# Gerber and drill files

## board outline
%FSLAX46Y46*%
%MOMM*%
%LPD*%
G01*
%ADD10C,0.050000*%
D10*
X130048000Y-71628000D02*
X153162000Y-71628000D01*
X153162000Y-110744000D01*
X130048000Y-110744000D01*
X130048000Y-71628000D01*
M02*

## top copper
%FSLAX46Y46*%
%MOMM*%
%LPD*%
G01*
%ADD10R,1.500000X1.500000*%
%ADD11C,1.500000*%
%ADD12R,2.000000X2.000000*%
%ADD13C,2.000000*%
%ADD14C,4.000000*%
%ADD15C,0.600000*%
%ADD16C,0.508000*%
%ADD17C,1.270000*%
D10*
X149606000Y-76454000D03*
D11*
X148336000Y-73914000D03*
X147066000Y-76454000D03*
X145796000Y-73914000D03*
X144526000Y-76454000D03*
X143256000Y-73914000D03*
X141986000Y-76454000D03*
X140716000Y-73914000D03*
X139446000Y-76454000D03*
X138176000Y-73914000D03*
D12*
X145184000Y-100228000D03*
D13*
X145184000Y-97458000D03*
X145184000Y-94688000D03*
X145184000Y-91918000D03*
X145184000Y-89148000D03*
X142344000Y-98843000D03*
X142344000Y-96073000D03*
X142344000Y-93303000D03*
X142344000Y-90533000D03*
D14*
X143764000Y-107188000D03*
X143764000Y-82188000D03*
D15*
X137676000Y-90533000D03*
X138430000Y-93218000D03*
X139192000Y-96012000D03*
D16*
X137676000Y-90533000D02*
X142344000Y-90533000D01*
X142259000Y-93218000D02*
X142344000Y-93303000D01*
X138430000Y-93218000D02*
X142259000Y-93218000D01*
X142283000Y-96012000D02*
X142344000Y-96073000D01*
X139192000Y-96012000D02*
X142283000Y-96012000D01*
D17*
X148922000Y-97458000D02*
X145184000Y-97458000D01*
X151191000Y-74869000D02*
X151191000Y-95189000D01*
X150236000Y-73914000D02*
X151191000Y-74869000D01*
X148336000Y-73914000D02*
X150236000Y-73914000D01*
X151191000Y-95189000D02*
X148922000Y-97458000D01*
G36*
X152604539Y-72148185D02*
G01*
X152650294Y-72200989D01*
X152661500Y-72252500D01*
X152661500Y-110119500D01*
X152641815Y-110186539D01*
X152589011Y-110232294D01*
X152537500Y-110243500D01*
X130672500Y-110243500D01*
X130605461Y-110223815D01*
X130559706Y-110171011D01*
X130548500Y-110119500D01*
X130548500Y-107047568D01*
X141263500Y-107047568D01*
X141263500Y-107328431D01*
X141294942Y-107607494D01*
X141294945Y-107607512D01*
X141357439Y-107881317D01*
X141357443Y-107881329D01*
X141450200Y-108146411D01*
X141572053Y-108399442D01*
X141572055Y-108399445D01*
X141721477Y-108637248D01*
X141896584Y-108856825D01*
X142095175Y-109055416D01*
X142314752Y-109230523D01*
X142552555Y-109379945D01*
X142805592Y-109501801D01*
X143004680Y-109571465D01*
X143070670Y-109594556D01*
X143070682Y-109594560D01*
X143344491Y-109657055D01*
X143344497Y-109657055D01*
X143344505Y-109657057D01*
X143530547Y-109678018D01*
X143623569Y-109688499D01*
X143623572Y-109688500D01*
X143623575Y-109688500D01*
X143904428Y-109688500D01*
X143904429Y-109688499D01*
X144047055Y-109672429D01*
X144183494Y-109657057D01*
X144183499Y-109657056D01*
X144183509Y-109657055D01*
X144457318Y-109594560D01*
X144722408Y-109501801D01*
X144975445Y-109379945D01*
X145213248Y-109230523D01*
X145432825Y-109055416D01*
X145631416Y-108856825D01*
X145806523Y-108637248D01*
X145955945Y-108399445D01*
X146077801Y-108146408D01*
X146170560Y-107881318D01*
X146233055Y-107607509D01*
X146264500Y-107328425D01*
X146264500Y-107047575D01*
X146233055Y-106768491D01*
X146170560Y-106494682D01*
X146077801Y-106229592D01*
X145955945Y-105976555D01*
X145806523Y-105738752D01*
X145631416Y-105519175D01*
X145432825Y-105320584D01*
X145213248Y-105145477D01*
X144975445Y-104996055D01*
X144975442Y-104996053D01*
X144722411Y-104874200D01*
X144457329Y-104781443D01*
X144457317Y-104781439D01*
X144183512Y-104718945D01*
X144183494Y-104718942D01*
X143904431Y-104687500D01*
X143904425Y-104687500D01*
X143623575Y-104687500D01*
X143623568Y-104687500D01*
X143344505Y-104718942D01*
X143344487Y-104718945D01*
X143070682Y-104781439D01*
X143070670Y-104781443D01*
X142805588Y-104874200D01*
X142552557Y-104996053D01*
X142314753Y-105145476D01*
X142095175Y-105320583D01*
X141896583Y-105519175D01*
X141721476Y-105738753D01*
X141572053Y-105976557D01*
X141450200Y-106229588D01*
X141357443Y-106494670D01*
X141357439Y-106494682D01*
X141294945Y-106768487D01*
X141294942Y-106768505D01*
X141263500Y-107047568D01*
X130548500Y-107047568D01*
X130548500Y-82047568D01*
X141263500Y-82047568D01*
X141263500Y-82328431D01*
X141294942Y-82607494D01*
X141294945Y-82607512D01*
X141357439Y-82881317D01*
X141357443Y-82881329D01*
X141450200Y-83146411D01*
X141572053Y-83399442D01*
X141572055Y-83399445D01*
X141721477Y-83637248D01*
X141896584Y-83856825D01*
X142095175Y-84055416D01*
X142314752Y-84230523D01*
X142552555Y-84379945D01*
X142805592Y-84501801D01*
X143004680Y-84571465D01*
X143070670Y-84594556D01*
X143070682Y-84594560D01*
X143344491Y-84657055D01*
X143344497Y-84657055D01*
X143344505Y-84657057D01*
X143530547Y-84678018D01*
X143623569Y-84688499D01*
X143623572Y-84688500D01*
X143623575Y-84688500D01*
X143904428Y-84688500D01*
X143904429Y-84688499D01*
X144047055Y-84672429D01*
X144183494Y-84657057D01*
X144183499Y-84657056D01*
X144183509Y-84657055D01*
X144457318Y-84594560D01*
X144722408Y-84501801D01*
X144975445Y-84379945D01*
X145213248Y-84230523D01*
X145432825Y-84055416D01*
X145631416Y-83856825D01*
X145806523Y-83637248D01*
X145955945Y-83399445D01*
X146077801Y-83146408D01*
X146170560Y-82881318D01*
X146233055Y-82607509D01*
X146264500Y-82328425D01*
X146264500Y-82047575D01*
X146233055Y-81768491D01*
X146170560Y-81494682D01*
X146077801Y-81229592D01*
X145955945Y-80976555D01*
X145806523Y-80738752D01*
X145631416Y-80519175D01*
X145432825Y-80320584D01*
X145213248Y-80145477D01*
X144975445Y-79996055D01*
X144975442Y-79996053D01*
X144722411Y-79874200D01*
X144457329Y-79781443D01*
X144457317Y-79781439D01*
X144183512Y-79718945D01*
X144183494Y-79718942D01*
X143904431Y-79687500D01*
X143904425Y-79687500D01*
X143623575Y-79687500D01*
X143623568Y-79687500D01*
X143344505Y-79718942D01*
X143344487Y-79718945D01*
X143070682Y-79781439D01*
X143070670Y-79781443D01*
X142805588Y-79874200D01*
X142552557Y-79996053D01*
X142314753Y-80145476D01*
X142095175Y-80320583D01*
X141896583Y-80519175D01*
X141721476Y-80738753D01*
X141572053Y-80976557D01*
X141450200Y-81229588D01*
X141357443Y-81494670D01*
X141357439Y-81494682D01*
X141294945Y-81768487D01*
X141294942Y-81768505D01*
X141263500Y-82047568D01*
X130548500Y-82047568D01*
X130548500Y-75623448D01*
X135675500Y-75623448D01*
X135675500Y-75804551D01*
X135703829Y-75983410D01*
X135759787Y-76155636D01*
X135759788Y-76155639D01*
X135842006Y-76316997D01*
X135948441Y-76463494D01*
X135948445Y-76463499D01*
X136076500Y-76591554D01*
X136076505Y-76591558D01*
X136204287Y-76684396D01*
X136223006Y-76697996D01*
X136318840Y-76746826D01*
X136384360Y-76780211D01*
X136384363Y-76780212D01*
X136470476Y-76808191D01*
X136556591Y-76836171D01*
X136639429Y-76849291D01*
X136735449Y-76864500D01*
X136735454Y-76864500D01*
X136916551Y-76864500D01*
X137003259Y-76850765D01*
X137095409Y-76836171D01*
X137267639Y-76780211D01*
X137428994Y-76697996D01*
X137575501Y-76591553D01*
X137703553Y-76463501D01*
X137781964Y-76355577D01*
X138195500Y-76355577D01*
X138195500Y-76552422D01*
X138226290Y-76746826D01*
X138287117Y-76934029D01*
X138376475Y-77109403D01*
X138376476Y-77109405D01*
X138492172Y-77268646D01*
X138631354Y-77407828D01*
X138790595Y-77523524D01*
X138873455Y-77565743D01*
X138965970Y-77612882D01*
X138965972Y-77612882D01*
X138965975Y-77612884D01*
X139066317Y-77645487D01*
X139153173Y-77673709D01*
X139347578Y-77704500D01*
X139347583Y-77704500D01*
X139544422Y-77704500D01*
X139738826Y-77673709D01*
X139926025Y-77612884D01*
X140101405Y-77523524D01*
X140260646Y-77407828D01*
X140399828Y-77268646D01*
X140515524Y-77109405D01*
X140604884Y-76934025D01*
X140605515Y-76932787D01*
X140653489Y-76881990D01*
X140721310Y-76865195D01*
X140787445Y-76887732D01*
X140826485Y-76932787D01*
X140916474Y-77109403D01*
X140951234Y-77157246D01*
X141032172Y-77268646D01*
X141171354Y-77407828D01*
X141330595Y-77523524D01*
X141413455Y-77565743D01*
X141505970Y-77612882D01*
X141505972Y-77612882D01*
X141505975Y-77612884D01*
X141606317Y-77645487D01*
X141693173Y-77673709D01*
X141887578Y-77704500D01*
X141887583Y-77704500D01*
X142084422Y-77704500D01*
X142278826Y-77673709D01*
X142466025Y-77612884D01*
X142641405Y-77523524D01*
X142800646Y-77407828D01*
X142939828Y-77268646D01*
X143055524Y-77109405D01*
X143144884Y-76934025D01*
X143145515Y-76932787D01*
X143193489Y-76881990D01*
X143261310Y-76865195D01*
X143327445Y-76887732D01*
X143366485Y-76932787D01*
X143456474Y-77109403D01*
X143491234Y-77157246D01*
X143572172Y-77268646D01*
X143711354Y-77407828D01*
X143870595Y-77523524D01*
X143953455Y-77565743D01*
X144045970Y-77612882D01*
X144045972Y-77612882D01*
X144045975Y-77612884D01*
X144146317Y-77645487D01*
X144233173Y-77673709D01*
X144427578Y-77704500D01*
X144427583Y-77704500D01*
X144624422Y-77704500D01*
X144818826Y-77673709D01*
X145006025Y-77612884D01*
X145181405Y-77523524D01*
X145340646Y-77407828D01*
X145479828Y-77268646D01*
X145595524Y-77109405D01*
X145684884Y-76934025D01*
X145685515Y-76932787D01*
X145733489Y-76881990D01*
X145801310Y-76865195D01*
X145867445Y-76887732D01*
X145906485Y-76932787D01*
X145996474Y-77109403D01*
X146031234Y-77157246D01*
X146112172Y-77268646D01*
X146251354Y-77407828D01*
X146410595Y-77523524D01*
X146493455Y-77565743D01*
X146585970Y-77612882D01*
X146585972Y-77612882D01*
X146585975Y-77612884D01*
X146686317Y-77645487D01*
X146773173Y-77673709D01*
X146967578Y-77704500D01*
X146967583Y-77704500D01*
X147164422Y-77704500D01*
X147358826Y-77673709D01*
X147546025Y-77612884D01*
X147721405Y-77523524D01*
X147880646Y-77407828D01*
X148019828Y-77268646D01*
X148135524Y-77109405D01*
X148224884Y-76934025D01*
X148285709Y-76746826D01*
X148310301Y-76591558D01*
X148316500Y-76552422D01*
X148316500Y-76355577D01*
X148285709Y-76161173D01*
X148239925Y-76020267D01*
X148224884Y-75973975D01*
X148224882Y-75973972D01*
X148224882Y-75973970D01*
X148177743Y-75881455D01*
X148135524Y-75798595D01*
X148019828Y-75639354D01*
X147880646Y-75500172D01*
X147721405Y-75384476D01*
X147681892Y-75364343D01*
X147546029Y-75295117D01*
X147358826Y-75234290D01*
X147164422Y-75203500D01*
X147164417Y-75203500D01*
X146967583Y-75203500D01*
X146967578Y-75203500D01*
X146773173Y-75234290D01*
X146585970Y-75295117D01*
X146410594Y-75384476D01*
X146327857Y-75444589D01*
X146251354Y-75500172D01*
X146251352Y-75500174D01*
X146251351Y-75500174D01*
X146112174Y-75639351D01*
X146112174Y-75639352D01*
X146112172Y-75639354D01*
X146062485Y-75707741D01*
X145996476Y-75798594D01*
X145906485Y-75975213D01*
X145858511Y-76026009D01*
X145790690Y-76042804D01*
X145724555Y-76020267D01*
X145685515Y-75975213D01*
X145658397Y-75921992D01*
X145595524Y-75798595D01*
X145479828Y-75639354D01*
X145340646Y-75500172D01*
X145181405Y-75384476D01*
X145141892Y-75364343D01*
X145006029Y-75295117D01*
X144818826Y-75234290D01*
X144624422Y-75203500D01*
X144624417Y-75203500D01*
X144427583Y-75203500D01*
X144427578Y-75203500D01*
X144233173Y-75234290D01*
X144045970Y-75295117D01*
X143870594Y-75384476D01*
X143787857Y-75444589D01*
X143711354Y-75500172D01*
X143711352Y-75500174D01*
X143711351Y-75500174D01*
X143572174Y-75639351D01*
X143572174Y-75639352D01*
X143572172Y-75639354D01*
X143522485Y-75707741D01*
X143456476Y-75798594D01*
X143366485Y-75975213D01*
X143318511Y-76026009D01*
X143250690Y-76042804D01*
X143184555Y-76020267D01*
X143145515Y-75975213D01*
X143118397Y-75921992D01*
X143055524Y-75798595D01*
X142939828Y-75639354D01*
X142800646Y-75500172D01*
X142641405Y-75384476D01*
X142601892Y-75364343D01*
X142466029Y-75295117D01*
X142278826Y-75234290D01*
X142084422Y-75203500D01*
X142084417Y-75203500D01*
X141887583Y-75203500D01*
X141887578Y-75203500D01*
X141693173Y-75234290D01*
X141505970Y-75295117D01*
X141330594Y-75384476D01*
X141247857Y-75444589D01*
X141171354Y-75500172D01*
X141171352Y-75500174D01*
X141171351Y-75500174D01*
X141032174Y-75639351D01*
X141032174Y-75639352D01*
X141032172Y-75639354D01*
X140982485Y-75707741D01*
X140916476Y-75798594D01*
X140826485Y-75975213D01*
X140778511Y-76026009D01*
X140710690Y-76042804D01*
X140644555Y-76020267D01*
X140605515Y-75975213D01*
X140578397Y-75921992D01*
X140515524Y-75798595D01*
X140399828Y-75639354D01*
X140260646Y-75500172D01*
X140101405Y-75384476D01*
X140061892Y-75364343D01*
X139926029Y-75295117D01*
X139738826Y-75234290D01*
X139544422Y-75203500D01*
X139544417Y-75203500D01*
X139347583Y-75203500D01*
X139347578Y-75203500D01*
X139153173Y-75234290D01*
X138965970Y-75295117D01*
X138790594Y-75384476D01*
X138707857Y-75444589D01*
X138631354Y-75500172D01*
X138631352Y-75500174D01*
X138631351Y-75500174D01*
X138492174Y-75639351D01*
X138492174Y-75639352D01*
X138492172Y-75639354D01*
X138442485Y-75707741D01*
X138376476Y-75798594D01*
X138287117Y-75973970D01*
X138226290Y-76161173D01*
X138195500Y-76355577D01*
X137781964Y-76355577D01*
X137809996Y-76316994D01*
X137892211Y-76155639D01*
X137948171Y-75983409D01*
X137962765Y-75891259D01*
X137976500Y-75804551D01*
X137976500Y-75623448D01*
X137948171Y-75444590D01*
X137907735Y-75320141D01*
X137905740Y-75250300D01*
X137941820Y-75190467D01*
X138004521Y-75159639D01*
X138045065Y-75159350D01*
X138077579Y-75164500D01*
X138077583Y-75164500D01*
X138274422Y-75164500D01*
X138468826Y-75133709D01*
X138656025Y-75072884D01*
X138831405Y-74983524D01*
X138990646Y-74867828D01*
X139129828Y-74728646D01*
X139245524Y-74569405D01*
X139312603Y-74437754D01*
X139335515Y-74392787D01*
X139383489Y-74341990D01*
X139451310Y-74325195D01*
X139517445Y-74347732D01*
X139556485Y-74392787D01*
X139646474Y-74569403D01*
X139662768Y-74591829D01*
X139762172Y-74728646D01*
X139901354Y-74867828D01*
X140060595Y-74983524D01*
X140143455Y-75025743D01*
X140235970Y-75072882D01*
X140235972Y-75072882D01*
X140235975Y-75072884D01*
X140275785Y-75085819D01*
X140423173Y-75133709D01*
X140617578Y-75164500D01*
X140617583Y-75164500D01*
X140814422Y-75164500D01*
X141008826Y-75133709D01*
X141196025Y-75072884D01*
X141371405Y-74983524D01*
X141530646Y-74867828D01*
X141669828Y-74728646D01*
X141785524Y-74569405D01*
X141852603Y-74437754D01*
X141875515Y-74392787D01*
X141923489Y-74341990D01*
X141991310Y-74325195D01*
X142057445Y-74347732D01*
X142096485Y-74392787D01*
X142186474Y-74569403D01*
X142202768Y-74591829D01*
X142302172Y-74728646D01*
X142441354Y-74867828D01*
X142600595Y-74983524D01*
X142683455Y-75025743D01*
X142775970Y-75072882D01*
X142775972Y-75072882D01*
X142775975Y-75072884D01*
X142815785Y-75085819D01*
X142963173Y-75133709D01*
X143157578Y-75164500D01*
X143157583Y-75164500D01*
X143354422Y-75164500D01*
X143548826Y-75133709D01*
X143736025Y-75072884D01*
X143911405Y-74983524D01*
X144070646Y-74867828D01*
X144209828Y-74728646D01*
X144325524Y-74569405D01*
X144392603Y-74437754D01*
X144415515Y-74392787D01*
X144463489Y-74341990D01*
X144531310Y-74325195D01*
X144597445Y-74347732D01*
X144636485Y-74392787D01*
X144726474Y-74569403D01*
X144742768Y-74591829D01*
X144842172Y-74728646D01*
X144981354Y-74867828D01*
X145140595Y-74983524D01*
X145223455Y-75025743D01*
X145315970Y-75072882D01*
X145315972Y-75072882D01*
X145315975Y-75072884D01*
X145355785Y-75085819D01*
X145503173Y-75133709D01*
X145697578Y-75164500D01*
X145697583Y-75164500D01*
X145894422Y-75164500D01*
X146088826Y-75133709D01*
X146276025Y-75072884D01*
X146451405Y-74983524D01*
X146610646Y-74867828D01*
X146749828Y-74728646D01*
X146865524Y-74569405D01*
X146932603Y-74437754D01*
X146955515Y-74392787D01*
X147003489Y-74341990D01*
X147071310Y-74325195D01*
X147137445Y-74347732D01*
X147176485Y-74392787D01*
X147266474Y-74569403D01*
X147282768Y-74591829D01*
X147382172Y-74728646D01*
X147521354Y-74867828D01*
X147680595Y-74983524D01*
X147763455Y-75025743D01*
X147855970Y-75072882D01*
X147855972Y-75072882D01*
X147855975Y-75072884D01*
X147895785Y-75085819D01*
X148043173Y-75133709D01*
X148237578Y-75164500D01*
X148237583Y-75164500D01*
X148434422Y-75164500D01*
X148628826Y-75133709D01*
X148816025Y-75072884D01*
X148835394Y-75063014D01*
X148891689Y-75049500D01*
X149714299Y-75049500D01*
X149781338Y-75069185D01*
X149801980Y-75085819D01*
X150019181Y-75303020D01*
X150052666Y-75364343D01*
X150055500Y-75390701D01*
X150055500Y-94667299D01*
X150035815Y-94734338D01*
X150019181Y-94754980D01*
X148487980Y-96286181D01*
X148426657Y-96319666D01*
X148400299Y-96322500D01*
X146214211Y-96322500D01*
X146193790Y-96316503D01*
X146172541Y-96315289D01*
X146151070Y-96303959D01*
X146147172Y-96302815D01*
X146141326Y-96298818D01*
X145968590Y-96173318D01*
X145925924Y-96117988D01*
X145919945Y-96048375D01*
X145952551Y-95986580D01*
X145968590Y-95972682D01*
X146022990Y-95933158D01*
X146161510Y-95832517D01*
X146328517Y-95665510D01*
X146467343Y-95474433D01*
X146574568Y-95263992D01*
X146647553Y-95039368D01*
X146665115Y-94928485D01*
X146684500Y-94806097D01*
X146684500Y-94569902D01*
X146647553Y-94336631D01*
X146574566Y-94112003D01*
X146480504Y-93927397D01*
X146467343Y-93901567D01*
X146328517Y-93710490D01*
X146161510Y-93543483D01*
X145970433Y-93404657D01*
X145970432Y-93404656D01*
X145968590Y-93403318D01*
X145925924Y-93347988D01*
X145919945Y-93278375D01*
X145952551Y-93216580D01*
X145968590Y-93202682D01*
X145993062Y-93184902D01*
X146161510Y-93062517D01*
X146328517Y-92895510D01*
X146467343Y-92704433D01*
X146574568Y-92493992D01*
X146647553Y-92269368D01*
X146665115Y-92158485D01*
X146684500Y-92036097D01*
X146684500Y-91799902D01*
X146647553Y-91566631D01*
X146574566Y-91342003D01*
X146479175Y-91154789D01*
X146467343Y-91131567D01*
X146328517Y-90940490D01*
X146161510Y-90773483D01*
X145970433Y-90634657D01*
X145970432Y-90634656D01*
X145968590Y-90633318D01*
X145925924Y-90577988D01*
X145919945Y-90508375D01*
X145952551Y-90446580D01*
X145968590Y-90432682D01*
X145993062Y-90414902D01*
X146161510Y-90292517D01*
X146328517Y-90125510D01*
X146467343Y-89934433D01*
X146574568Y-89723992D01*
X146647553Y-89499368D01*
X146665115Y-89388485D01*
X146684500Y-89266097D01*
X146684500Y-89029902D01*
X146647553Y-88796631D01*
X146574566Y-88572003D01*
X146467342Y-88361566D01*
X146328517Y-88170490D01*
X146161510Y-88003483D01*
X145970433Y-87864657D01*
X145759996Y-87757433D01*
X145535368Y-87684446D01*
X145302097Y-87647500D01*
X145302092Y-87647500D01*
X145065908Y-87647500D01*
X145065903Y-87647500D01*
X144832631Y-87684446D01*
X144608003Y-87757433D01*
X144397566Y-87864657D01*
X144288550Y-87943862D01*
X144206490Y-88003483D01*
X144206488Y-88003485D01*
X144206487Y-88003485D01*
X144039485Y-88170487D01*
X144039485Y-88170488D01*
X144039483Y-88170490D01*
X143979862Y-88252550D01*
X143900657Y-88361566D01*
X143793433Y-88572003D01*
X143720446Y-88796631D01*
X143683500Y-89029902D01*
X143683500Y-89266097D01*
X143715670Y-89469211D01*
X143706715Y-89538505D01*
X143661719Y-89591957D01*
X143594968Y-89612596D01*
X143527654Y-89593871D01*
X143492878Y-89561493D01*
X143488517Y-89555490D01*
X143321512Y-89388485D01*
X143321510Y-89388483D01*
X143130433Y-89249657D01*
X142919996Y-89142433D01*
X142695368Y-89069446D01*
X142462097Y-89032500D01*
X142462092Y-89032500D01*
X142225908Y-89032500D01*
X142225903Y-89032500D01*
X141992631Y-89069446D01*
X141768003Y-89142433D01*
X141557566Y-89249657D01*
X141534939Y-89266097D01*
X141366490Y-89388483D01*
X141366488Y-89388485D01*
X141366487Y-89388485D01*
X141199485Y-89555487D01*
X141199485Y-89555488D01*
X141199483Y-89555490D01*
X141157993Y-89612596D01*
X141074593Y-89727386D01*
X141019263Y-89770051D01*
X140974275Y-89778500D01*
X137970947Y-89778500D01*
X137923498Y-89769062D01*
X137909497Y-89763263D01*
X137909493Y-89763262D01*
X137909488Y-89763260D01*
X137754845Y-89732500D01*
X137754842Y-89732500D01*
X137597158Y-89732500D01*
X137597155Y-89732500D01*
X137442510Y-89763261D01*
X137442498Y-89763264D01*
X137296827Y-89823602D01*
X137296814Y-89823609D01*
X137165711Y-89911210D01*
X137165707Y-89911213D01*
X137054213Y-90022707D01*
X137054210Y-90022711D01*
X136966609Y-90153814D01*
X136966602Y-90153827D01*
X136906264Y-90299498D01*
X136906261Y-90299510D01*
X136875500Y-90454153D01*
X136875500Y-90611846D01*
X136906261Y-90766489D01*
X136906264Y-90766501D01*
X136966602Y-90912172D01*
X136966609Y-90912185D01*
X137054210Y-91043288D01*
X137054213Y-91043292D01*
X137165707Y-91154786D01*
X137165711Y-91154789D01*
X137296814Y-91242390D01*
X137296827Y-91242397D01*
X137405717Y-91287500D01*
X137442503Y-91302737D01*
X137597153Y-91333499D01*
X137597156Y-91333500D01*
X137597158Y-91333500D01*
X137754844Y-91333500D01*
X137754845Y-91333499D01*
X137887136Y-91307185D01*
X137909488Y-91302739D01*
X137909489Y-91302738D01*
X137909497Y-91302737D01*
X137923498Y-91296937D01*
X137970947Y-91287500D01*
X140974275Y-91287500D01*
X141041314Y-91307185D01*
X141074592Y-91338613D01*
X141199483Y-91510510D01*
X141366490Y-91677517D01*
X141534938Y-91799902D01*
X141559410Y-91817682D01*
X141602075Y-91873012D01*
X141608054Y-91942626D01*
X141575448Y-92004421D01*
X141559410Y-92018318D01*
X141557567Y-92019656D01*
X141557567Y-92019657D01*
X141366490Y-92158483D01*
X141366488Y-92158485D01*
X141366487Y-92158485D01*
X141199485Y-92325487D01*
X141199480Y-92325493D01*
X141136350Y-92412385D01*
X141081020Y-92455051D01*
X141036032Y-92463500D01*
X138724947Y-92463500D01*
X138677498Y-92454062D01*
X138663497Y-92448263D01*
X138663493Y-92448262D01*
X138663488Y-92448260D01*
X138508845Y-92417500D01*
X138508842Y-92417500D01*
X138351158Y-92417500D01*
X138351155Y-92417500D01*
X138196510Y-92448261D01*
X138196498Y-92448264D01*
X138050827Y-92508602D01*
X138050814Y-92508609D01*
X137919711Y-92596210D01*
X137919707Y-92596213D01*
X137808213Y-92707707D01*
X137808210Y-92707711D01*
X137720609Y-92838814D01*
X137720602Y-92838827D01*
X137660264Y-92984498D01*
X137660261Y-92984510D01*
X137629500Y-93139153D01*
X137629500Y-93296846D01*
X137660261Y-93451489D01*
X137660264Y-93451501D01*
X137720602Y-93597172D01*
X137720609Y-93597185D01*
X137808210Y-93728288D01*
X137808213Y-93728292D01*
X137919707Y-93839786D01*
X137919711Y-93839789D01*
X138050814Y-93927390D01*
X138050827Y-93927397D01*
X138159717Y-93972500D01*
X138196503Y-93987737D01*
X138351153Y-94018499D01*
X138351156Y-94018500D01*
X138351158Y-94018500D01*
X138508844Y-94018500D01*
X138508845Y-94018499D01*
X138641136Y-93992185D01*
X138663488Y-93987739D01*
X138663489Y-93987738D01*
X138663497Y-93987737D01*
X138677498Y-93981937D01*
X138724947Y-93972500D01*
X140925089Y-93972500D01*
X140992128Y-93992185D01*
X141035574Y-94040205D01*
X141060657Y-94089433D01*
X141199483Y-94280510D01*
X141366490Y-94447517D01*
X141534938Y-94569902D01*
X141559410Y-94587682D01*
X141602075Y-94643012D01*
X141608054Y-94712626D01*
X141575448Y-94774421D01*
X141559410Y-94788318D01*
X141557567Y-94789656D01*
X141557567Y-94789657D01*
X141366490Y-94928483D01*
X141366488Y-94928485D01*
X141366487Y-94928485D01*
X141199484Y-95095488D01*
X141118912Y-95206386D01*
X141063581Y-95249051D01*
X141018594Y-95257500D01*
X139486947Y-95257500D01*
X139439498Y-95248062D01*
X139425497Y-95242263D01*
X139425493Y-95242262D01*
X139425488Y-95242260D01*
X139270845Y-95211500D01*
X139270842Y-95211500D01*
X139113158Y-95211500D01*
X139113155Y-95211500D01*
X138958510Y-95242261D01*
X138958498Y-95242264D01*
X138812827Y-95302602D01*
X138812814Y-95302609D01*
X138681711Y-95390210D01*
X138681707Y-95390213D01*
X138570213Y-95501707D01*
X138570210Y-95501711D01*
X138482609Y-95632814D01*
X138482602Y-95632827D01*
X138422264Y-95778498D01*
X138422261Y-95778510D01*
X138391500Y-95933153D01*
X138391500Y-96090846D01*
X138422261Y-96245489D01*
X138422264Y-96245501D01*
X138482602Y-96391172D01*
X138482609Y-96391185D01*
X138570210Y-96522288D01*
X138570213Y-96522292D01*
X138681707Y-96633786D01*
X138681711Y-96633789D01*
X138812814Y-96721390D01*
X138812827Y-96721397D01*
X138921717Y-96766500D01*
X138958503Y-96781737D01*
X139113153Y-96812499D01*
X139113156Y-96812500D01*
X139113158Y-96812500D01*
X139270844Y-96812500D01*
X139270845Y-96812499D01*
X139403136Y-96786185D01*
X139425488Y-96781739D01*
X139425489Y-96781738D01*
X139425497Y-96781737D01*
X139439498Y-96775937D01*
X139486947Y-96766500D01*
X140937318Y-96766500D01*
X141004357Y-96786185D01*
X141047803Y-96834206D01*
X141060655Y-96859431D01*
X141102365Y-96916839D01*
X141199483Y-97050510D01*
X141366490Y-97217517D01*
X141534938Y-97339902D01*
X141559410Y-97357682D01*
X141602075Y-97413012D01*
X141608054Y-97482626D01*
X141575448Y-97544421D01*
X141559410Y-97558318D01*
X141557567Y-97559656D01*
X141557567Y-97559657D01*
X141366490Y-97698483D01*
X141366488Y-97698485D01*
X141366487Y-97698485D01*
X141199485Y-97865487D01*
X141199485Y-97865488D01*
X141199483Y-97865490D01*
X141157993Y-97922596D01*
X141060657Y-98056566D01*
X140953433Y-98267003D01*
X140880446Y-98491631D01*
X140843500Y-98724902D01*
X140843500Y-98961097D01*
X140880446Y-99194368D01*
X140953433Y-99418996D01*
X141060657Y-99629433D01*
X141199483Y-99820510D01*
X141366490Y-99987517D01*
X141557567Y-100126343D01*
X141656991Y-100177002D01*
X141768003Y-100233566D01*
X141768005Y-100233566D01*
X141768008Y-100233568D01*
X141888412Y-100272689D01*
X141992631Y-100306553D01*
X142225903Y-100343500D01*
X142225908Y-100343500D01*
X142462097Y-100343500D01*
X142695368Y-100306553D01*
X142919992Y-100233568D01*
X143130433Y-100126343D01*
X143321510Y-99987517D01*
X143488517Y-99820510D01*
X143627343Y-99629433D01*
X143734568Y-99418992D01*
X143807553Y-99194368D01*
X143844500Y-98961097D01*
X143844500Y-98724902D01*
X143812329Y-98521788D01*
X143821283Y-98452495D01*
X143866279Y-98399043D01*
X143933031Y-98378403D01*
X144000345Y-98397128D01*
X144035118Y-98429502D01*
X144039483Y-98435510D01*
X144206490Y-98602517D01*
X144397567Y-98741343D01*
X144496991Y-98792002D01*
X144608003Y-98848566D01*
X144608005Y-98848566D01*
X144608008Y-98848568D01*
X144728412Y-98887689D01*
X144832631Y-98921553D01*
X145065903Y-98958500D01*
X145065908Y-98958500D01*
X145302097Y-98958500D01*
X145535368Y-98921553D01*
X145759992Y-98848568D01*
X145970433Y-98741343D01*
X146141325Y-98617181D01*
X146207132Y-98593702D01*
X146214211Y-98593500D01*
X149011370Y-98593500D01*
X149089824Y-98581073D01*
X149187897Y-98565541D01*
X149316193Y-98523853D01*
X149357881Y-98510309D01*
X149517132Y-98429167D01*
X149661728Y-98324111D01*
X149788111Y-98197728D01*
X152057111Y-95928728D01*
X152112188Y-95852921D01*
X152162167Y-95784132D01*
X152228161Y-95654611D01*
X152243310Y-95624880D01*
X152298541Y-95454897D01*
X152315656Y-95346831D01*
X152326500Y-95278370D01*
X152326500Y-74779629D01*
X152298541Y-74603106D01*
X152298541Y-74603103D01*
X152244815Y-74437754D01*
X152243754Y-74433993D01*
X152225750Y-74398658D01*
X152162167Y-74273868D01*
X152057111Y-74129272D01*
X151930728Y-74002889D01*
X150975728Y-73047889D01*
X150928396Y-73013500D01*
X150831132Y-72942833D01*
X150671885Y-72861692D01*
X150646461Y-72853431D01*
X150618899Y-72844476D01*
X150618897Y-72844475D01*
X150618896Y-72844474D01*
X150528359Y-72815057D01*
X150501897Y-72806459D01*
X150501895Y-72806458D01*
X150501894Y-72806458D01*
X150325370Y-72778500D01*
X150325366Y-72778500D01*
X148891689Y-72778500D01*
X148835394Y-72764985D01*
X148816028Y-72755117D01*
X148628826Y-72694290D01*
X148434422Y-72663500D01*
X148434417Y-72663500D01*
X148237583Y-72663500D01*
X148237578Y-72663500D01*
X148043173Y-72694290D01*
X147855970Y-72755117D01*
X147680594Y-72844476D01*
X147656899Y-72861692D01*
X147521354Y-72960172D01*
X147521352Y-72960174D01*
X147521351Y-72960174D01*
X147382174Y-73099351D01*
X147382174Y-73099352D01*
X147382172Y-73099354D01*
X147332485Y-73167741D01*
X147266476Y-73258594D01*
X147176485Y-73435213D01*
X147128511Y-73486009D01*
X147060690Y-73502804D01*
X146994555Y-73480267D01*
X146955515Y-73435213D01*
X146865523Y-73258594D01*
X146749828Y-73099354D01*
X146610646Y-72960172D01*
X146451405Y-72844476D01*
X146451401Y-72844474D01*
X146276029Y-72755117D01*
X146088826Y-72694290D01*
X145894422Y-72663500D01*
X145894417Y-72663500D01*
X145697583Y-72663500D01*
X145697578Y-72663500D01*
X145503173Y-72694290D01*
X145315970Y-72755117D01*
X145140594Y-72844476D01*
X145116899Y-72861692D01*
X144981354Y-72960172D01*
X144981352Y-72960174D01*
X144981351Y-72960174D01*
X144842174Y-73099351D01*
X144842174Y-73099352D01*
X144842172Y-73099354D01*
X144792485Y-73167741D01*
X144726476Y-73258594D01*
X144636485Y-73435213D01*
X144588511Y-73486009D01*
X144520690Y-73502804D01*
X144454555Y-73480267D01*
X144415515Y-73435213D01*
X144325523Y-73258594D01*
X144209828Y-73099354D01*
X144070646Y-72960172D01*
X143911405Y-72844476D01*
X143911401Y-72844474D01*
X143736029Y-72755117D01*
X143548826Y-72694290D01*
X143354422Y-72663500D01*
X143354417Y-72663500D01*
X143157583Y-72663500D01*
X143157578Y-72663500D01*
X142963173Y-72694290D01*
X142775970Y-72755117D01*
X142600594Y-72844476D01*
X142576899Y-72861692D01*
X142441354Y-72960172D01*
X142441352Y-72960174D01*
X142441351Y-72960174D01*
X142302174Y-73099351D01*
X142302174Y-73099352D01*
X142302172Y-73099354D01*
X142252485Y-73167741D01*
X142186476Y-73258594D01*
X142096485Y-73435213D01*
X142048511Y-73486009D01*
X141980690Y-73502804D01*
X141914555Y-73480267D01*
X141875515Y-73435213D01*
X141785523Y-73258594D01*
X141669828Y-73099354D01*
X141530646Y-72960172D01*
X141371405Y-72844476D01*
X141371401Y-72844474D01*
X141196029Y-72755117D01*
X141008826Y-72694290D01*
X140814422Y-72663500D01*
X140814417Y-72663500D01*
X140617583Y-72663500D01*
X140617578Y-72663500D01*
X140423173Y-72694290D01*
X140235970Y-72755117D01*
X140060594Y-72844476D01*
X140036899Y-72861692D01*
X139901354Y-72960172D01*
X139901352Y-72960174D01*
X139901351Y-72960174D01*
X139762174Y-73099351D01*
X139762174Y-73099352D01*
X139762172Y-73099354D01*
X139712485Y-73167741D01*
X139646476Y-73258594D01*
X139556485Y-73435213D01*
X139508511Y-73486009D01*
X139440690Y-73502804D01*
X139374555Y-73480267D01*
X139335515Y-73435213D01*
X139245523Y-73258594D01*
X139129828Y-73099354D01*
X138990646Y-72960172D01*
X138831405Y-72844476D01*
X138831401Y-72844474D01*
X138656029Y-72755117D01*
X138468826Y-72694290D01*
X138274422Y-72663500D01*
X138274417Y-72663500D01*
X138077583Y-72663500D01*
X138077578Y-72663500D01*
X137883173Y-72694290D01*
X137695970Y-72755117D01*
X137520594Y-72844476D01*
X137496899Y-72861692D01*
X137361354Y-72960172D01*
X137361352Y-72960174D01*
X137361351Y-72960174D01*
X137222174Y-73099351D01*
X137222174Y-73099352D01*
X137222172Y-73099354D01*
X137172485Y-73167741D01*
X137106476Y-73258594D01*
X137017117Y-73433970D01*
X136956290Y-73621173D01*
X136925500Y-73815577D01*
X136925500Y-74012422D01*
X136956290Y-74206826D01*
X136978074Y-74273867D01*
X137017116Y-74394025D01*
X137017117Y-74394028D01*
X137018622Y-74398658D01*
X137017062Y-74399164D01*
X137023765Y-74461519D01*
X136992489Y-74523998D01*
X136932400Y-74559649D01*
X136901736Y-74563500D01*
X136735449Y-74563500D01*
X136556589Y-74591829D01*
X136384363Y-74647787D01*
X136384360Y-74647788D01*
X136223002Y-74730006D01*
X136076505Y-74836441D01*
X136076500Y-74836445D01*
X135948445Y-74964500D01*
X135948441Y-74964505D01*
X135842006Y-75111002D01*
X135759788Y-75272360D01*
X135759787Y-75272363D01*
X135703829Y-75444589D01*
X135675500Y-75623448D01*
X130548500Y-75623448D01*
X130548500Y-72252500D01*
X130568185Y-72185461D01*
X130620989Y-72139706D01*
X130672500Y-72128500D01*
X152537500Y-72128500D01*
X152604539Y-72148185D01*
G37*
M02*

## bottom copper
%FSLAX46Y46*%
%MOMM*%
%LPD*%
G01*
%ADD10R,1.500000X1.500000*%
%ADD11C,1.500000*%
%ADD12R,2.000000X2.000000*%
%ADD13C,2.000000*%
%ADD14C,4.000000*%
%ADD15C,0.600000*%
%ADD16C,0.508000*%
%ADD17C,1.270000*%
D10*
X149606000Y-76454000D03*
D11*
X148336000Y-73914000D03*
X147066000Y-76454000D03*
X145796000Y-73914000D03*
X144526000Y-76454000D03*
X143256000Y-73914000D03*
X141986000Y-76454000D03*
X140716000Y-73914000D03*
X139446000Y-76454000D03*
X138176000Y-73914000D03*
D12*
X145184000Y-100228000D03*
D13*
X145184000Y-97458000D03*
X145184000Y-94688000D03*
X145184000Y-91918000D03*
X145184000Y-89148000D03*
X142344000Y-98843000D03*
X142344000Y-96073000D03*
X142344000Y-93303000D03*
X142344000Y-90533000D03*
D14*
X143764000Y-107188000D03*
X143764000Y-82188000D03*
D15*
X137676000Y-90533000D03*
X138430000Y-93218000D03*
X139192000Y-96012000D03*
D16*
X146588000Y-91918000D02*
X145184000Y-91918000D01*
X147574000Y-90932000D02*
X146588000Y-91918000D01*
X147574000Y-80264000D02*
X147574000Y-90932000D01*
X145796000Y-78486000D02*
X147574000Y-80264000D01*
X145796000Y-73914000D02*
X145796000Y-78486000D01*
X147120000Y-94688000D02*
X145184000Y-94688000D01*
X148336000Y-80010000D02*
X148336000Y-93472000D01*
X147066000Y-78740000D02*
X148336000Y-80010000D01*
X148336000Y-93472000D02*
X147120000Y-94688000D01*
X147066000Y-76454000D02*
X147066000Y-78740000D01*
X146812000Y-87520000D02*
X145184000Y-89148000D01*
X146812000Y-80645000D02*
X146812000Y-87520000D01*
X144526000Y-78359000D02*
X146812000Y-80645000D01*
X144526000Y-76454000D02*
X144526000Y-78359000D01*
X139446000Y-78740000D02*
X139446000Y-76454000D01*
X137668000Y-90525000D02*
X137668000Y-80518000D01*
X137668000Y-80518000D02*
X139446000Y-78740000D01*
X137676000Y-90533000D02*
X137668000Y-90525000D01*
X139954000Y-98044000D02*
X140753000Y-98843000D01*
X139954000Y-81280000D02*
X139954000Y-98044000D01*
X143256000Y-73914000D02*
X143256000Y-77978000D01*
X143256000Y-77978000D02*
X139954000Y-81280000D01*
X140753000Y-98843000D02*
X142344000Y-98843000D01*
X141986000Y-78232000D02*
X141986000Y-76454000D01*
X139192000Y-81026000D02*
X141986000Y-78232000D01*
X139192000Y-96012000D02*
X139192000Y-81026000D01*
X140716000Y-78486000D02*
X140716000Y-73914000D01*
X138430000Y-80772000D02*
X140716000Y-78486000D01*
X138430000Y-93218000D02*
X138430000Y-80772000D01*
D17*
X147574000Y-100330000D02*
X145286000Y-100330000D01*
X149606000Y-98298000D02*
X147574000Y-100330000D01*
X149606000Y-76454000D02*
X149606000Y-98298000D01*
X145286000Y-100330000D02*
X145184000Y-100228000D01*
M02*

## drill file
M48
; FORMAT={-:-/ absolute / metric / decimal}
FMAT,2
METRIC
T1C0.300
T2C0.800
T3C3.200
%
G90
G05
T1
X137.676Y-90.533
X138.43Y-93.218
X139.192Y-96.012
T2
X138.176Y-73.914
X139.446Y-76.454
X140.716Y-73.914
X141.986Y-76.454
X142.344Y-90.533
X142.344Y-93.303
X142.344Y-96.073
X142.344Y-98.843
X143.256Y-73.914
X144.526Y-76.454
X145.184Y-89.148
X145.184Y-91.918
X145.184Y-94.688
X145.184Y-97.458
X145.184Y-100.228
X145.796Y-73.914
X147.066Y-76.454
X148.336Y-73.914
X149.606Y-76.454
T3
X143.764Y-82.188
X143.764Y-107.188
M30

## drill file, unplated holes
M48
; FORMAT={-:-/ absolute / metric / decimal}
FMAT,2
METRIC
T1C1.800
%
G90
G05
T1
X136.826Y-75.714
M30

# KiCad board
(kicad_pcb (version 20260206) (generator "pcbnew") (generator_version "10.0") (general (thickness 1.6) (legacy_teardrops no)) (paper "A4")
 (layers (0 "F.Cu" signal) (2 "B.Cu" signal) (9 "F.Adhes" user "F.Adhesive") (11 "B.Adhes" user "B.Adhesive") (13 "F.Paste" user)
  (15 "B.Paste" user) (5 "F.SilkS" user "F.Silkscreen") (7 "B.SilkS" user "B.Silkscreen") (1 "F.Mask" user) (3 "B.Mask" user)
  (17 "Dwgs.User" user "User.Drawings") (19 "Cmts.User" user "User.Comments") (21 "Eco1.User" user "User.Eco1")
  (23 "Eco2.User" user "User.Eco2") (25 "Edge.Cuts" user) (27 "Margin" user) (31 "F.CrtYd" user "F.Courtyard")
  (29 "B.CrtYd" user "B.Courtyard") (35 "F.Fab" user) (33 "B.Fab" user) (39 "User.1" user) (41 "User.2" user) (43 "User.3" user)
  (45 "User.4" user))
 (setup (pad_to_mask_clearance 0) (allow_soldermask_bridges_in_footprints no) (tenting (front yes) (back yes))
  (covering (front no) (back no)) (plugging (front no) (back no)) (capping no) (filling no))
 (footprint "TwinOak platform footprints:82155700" (layer "F.Cu") (at 149.606 76.454 180)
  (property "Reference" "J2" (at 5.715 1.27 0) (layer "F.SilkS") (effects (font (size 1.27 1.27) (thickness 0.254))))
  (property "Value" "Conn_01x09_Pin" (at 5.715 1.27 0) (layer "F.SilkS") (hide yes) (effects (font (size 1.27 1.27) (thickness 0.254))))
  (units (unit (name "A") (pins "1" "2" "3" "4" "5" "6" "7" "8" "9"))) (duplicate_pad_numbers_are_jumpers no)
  (pad "" np_thru_hole circle (at 12.78 0.74 180) (size 1.8 1.8) (drill 1.8) (layers "*.Cu" "*.Mask"))
  (pad "1" thru_hole rect (at 0 0 180) (size 1.5 1.5) (drill 0.8) (layers "*.Cu" "*.Mask") (remove_unused_layers no) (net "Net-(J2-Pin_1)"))
  (pad "2" thru_hole circle (at 1.27 2.54 180) (size 1.5 1.5) (drill 0.8) (layers "*.Cu" "*.Mask") (remove_unused_layers no)
   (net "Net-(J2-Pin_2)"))
  (pad "3" thru_hole circle (at 2.54 0 180) (size 1.5 1.5) (drill 0.8) (layers "*.Cu" "*.Mask") (remove_unused_layers no)
   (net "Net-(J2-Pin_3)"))
  (pad "4" thru_hole circle (at 3.81 2.54 180) (size 1.5 1.5) (drill 0.8) (layers "*.Cu" "*.Mask") (remove_unused_layers no)
   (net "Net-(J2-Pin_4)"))
  (pad "5" thru_hole circle (at 5.08 0 180) (size 1.5 1.5) (drill 0.8) (layers "*.Cu" "*.Mask") (remove_unused_layers no)
   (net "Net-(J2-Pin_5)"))
  (pad "6" thru_hole circle (at 6.35 2.54 180) (size 1.5 1.5) (drill 0.8) (layers "*.Cu" "*.Mask") (remove_unused_layers no)
   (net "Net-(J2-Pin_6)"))
  (pad "7" thru_hole circle (at 7.62 0 180) (size 1.5 1.5) (drill 0.8) (layers "*.Cu" "*.Mask") (remove_unused_layers no)
   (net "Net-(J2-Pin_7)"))
  (pad "8" thru_hole circle (at 8.89 2.54 180) (size 1.5 1.5) (drill 0.8) (layers "*.Cu" "*.Mask") (remove_unused_layers no)
   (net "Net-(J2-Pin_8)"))
  (pad "9" thru_hole circle (at 10.16 0 180) (size 1.5 1.5) (drill 0.8) (layers "*.Cu" "*.Mask") (remove_unused_layers no)
   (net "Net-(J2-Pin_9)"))
  (pad "10" thru_hole circle (at 11.43 2.54 180) (size 1.5 1.5) (drill 0.8) (layers "*.Cu" "*.Mask") (remove_unused_layers no)))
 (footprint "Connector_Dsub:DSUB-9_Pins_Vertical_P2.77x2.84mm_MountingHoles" (layer "B.Cu") (at 145.184 100.228 90)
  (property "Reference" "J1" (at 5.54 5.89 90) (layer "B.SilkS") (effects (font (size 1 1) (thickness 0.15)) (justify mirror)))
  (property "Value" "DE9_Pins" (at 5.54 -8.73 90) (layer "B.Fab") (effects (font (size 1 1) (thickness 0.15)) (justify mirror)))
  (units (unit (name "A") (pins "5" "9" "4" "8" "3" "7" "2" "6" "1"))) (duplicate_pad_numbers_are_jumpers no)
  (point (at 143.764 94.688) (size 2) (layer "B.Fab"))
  (pad "1" thru_hole rect (at 0 0 90) (size 2 2) (drill 0.8) (layers "*.Cu" "*.Mask") (remove_unused_layers no) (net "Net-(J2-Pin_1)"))
  (pad "2" thru_hole circle (at 2.77 0 90) (size 2 2) (drill 0.8) (layers "*.Cu" "*.Mask") (remove_unused_layers no) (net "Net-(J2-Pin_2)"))
  (pad "3" thru_hole circle (at 5.54 0 90) (size 2 2) (drill 0.8) (layers "*.Cu" "*.Mask") (remove_unused_layers no) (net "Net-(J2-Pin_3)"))
  (pad "4" thru_hole circle (at 8.31 0 90) (size 2 2) (drill 0.8) (layers "*.Cu" "*.Mask") (remove_unused_layers no) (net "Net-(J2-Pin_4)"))
  (pad "5" thru_hole circle (at 11.08 0 90) (size 2 2) (drill 0.8) (layers "*.Cu" "*.Mask") (remove_unused_layers no) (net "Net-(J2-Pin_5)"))
  (pad "6" thru_hole circle (at 1.385 -2.84 90) (size 2 2) (drill 0.8) (layers "*.Cu" "*.Mask") (remove_unused_layers no)
   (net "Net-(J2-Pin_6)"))
  (pad "7" thru_hole circle (at 4.155 -2.84 90) (size 2 2) (drill 0.8) (layers "*.Cu" "*.Mask") (remove_unused_layers no)
   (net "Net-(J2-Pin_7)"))
  (pad "8" thru_hole circle (at 6.925 -2.84 90) (size 2 2) (drill 0.8) (layers "*.Cu" "*.Mask") (remove_unused_layers no)
   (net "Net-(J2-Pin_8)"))
  (pad "9" thru_hole circle (at 9.695 -2.84 90) (size 2 2) (drill 0.8) (layers "*.Cu" "*.Mask") (remove_unused_layers no)
   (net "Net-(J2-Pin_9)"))
  (pad "SH" thru_hole circle (at -6.96 -1.42 90) (size 4 4) (drill 3.2) (layers "*.Cu" "*.Mask") (remove_unused_layers no))
  (pad "SH" thru_hole circle (at 18.04 -1.42 90) (size 4 4) (drill 3.2) (layers "*.Cu" "*.Mask") (remove_unused_layers no)))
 (gr_rect (start 130.048 71.628) (end 153.162 110.744) (stroke (width 0.05) (type default)) (fill no) (layer "Edge.Cuts"))
 (segment (start 149.606 98.298) (end 147.574 100.33) (width 1.27) (layer "B.Cu") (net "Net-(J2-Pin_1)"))
 (segment (start 147.574 100.33) (end 145.286 100.33) (width 1.27) (layer "B.Cu") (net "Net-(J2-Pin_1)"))
 (segment (start 145.286 100.33) (end 145.184 100.228) (width 1.27) (layer "B.Cu") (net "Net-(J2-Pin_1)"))
 (segment (start 149.606 76.454) (end 149.606 98.298) (width 1.27) (layer "B.Cu") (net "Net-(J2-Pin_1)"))
 (segment (start 148.922 97.458) (end 145.184 97.458) (width 1.27) (layer "F.Cu") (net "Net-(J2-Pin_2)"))
 (segment (start 151.191 74.869) (end 151.191 95.189) (width 1.27) (layer "F.Cu") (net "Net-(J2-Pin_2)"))
 (segment (start 148.336 73.914) (end 150.236 73.914) (width 1.27) (layer "F.Cu") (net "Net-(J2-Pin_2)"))
 (segment (start 151.191 95.189) (end 148.922 97.458) (width 1.27) (layer "F.Cu") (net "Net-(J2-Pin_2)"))
 (segment (start 150.236 73.914) (end 151.191 74.869) (width 1.27) (layer "F.Cu") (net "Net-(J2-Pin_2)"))
 (segment (start 148.336 80.01) (end 148.336 93.472) (width 0.508) (layer "B.Cu") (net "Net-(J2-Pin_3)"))
 (segment (start 148.336 93.472) (end 147.12 94.688) (width 0.508) (layer "B.Cu") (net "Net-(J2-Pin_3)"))
 (segment (start 147.12 94.688) (end 145.184 94.688) (width 0.508) (layer "B.Cu") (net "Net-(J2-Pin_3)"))
 (segment (start 147.066 76.454) (end 147.066 78.74) (width 0.508) (layer "B.Cu") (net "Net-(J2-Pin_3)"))
 (segment (start 147.066 78.74) (end 148.336 80.01) (width 0.508) (layer "B.Cu") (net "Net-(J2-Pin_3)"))
 (segment (start 146.588 91.918) (end 145.184 91.918) (width 0.508) (layer "B.Cu") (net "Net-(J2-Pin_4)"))
 (segment (start 147.574 90.932) (end 146.588 91.918) (width 0.508) (layer "B.Cu") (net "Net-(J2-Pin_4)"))
 (segment (start 145.796 78.486) (end 147.574 80.264) (width 0.508) (layer "B.Cu") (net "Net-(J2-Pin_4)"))
 (segment (start 145.796 73.914) (end 145.796 78.486) (width 0.508) (layer "B.Cu") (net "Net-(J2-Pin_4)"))
 (segment (start 147.574 80.264) (end 147.574 90.932) (width 0.508) (layer "B.Cu") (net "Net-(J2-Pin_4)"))
 (segment (start 144.526 78.359) (end 146.812 80.645) (width 0.508) (layer "B.Cu") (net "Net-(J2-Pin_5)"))
 (segment (start 146.812 80.645) (end 146.812 87.52) (width 0.508) (layer "B.Cu") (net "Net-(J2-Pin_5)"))
 (segment (start 146.812 87.52) (end 145.184 89.148) (width 0.508) (layer "B.Cu") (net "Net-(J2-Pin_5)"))
 (segment (start 144.526 76.454) (end 144.526 78.359) (width 0.508) (layer "B.Cu") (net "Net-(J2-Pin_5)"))
 (segment (start 143.256 73.914) (end 143.256 77.978) (width 0.508) (layer "B.Cu") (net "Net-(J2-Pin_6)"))
 (segment (start 139.954 81.28) (end 139.954 98.044) (width 0.508) (layer "B.Cu") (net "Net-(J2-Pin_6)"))
 (segment (start 143.256 77.978) (end 139.954 81.28) (width 0.508) (layer "B.Cu") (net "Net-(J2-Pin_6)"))
 (segment (start 140.753 98.843) (end 142.344 98.843) (width 0.508) (layer "B.Cu") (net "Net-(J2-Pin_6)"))
 (segment (start 139.954 98.044) (end 140.753 98.843) (width 0.508) (layer "B.Cu") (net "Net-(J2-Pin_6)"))
 (segment (start 139.192 96.012) (end 142.283 96.012) (width 0.508) (layer "F.Cu") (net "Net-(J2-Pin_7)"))
 (segment (start 142.283 96.012) (end 142.344 96.073) (width 0.508) (layer "F.Cu") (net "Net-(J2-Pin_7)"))
 (via (at 139.192 96.012) (size 0.6) (drill 0.3) (layers "F.Cu" "B.Cu") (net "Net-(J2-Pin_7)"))
 (segment (start 139.192 81.026) (end 141.986 78.232) (width 0.508) (layer "B.Cu") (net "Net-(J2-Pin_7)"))
 (segment (start 141.986 78.232) (end 141.986 76.454) (width 0.508) (layer "B.Cu") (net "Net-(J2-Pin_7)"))
 (segment (start 139.192 96.012) (end 139.192 81.026) (width 0.508) (layer "B.Cu") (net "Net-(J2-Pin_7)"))
 (segment (start 142.259 93.218) (end 142.344 93.303) (width 0.508) (layer "F.Cu") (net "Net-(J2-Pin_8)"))
 (segment (start 138.43 93.218) (end 142.259 93.218) (width 0.508) (layer "F.Cu") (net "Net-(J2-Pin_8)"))
 (via (at 138.43 93.218) (size 0.6) (drill 0.3) (layers "F.Cu" "B.Cu") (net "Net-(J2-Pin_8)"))
 (segment (start 138.43 93.218) (end 138.43 80.772) (width 0.508) (layer "B.Cu") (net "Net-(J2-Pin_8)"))
 (segment (start 138.43 80.772) (end 140.716 78.486) (width 0.508) (layer "B.Cu") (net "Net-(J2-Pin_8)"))
 (segment (start 140.716 78.486) (end 140.716 73.914) (width 0.508) (layer "B.Cu") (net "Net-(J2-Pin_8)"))
 (segment (start 137.676 90.533) (end 142.344 90.533) (width 0.508) (layer "F.Cu") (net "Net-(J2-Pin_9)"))
 (via (at 137.676 90.533) (size 0.6) (drill 0.3) (layers "F.Cu" "B.Cu") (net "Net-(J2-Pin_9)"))
 (segment (start 137.668 90.525) (end 137.668 80.518) (width 0.508) (layer "B.Cu") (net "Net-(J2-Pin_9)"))
 (segment (start 139.446 78.74) (end 139.446 76.454) (width 0.508) (layer "B.Cu") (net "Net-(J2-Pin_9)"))
 (segment (start 137.668 80.518) (end 139.446 78.74) (width 0.508) (layer "B.Cu") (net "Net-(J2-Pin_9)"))
 (segment (start 137.676 90.533) (end 137.668 90.525) (width 0.508) (layer "B.Cu") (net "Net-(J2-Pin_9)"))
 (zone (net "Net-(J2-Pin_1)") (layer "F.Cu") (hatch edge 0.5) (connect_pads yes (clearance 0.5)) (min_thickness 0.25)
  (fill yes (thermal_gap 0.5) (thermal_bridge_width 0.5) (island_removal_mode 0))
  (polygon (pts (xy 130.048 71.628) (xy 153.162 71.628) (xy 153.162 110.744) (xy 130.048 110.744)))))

